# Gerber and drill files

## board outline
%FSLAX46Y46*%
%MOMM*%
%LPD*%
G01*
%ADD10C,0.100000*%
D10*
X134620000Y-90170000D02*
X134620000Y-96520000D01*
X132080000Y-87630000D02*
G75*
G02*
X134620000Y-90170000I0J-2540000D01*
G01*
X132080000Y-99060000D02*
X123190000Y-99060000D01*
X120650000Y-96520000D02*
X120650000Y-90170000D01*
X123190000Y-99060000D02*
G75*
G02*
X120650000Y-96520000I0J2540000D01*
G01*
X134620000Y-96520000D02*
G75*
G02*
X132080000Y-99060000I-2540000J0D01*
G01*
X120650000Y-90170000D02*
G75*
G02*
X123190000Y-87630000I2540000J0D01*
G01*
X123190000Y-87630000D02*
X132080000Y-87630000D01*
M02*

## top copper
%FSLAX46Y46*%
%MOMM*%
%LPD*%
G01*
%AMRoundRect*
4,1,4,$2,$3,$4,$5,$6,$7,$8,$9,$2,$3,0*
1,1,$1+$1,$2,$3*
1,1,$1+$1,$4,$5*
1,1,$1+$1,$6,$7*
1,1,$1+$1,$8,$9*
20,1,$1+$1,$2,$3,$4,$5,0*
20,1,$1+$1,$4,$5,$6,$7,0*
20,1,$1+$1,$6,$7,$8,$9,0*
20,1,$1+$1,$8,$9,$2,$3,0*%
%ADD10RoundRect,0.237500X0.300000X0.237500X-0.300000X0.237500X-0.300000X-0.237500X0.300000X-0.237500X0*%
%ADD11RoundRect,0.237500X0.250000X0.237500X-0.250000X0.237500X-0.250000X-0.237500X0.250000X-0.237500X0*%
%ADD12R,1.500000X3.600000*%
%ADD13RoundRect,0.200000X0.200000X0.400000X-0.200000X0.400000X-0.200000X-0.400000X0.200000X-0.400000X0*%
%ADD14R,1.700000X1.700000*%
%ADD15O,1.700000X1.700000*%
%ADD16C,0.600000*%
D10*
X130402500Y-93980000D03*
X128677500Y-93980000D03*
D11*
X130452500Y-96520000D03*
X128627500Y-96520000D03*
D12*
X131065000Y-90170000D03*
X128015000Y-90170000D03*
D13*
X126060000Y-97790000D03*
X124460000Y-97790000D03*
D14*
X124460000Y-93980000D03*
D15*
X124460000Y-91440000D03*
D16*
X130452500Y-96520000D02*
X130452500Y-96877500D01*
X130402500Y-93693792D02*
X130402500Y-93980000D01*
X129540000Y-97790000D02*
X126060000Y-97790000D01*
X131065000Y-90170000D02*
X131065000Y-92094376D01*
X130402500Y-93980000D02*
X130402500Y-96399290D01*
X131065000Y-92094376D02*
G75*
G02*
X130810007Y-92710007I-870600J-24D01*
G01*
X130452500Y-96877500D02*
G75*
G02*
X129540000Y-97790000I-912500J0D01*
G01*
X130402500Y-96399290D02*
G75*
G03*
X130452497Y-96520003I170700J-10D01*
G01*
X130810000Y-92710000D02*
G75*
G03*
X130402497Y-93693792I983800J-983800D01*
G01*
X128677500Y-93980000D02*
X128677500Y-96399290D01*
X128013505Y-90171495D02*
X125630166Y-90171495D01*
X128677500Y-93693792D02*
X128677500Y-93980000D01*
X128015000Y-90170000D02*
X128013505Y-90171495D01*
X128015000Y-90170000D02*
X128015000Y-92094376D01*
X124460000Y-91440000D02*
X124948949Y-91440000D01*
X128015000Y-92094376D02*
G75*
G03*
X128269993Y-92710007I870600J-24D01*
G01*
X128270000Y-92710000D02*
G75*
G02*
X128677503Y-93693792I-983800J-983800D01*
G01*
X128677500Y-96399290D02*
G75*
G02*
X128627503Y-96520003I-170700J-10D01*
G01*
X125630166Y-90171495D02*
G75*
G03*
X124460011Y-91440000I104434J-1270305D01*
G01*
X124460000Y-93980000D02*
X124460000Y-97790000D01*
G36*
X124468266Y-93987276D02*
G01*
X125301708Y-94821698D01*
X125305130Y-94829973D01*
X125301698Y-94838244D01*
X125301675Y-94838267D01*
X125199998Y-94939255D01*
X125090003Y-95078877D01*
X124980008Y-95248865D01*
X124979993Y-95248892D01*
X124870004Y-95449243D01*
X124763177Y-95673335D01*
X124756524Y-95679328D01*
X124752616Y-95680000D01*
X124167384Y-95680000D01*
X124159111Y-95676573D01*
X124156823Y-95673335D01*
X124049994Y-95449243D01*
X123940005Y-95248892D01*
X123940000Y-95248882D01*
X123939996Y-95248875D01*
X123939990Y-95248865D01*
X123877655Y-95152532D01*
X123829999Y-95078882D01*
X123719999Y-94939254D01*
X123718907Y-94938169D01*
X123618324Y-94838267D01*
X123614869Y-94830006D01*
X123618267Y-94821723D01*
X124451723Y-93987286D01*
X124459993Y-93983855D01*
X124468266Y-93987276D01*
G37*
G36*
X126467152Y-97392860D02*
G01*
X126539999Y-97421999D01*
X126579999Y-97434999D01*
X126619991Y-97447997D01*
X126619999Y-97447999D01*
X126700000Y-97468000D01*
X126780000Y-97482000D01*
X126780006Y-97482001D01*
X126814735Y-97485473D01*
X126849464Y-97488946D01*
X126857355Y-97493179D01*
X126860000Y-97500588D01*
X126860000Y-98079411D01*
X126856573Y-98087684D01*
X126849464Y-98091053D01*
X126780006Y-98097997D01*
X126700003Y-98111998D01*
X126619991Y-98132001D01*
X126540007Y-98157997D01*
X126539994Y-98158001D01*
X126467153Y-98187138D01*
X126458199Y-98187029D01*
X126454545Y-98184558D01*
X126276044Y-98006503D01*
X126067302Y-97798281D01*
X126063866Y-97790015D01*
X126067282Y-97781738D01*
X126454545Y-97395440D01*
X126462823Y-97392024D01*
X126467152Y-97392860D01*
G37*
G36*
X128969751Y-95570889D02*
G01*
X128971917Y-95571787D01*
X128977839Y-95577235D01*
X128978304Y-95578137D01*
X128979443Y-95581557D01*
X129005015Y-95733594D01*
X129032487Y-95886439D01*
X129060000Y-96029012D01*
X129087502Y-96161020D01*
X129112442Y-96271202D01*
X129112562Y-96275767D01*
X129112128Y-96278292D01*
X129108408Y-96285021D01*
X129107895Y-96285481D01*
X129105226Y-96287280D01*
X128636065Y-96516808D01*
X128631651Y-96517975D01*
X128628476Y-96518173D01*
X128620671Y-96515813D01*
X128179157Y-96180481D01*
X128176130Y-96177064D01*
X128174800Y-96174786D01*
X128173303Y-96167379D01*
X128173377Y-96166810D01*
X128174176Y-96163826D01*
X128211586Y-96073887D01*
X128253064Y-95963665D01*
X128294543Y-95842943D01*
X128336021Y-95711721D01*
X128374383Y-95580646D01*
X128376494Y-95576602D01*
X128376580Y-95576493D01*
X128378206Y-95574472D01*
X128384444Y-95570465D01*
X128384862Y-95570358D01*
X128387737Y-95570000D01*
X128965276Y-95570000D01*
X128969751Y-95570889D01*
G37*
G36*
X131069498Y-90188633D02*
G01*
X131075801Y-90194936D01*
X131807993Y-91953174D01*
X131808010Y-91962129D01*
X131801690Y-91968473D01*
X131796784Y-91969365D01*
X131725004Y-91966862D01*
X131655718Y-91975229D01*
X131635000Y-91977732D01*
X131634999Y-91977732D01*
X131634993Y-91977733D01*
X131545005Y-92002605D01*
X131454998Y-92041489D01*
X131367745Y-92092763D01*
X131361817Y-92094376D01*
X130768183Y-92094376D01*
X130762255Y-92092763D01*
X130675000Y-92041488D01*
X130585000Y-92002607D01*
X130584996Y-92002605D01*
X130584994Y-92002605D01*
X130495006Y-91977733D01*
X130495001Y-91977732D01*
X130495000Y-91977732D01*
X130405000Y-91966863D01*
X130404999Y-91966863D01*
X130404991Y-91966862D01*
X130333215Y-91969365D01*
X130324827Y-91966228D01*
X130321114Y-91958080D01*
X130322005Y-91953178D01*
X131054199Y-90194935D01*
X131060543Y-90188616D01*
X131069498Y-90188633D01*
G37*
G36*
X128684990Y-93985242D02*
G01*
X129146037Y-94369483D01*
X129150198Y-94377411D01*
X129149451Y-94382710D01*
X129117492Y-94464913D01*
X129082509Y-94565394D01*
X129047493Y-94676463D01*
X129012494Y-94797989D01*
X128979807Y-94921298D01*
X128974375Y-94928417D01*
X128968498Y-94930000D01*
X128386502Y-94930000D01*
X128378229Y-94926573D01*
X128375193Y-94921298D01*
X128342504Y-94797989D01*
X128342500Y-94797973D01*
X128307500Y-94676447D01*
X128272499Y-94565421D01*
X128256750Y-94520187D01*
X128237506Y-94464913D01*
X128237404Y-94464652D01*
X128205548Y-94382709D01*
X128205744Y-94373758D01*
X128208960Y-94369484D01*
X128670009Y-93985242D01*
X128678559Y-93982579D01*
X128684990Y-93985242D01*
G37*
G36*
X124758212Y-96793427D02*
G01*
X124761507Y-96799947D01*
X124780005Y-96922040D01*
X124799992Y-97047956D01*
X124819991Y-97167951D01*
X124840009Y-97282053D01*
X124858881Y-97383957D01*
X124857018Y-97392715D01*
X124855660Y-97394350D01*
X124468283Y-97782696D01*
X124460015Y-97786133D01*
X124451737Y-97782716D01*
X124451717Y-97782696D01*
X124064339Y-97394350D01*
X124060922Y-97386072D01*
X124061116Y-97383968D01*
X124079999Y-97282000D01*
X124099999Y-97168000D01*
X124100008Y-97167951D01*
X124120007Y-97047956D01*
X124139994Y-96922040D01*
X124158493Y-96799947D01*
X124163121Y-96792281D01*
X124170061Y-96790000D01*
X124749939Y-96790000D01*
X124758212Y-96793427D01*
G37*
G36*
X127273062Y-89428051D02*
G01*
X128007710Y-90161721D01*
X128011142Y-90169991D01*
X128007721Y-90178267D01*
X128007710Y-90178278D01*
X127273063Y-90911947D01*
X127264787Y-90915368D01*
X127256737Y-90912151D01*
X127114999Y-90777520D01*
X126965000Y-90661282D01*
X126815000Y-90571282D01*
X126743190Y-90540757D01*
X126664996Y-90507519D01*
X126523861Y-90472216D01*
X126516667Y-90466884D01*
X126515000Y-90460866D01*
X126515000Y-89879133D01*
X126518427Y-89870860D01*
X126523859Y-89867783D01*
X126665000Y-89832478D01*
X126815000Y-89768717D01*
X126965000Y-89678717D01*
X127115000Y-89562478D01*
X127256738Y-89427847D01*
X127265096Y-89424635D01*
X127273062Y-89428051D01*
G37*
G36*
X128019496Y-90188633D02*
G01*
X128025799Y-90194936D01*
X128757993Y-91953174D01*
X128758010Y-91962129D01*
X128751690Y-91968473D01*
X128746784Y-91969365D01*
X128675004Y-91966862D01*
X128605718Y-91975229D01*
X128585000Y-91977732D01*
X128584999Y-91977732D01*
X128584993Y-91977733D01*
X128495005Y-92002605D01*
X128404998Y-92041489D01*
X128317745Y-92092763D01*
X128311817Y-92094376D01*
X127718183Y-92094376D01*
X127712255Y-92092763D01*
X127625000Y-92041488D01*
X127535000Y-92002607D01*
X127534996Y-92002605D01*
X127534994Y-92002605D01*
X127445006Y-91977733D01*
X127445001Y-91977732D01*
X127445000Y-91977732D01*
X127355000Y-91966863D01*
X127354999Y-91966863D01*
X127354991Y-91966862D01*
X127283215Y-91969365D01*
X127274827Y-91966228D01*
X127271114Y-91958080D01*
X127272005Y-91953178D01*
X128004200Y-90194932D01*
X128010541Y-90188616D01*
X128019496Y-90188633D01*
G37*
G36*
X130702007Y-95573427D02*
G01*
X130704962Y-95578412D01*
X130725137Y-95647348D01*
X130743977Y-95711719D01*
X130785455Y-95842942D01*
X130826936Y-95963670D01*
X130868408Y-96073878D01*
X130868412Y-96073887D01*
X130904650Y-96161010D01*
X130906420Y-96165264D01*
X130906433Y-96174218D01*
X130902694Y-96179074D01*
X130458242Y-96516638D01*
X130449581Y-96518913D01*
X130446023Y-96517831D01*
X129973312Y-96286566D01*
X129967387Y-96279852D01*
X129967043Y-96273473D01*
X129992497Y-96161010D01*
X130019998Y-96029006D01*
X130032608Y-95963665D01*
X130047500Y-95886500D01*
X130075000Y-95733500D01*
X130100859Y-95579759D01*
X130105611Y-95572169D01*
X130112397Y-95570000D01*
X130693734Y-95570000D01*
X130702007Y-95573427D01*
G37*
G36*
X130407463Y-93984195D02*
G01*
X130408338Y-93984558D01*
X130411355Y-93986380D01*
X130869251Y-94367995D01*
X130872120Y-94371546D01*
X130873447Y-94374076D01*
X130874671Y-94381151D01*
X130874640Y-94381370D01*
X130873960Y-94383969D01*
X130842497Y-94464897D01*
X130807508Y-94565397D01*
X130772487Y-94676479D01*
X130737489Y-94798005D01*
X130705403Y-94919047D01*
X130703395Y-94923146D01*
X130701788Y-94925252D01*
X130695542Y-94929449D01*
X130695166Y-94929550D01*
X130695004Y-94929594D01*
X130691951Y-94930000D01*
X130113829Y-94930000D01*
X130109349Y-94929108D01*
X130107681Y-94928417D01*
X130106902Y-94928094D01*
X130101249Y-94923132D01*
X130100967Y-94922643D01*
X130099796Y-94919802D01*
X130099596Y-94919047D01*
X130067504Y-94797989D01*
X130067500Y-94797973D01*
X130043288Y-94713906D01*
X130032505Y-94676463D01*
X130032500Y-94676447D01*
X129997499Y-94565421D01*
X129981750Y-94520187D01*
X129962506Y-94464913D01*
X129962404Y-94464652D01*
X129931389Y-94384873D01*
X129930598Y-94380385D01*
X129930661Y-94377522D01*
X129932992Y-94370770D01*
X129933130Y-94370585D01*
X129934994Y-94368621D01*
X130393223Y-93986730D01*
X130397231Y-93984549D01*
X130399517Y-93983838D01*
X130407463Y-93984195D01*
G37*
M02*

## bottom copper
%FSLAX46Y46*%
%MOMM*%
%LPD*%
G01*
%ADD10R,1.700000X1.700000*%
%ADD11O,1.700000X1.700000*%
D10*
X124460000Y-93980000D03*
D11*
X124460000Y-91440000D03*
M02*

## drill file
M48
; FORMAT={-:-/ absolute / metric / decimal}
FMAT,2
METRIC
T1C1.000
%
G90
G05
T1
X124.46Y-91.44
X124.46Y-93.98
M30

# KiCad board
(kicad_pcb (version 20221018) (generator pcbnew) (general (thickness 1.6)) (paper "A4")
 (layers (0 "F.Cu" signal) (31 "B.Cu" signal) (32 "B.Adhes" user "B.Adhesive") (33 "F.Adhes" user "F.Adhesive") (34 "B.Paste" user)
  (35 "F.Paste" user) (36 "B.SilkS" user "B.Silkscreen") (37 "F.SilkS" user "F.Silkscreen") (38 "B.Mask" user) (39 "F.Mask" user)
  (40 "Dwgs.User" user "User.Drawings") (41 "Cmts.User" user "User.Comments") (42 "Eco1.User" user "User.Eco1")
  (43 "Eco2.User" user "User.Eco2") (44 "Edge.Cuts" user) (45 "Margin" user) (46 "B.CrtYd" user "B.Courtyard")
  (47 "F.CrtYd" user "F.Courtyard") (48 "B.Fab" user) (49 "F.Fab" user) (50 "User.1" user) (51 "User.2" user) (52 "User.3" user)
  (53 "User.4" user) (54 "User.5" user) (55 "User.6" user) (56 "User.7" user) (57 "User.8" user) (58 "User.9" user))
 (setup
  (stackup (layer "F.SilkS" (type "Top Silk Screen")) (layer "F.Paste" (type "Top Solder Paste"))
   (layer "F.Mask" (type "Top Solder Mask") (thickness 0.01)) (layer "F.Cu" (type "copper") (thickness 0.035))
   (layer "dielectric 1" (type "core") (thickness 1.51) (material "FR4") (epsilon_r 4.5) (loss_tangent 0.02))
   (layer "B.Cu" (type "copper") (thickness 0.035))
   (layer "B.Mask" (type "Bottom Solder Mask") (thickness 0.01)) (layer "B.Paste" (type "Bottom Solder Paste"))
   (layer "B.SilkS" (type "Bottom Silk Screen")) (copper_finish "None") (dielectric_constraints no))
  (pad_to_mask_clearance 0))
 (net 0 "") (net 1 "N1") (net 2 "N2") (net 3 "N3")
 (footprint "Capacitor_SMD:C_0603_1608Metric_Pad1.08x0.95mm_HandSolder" (layer "F.Cu") (at 129.54 93.98 180)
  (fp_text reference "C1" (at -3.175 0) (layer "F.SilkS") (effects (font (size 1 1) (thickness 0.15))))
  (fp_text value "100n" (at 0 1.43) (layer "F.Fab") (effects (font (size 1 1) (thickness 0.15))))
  (pad "1" smd roundrect (at -0.8625 0 180) (size 1.075 0.95) (layers "F.Cu" "F.Paste" "F.Mask") (roundrect_rratio 0.25) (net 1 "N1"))
  (pad "2" smd roundrect (at 0.8625 0 180) (size 1.075 0.95) (layers "F.Cu" "F.Paste" "F.Mask") (roundrect_rratio 0.25) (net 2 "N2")))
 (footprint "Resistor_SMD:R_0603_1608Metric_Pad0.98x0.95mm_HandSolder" (layer "F.Cu") (at 129.54 96.52 180)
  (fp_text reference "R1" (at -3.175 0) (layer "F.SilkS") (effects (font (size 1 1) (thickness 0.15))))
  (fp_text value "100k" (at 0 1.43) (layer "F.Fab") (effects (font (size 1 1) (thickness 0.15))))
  (pad "1" smd roundrect (at -0.9125 0 180) (size 0.975 0.95) (layers "F.Cu" "F.Paste" "F.Mask") (roundrect_rratio 0.25) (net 1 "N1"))
  (pad "2" smd roundrect (at 0.9125 0 180) (size 0.975 0.95) (layers "F.Cu" "F.Paste" "F.Mask") (roundrect_rratio 0.25) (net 2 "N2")))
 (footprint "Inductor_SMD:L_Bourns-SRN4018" (layer "F.Cu") (at 129.54 90.17 180)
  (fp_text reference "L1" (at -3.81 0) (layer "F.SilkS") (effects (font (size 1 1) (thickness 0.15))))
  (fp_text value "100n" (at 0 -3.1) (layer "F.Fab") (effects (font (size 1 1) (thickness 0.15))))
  (pad "1" smd rect (at -1.525 0 180) (size 1.5 3.6) (layers "F.Cu" "F.Paste" "F.Mask") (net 1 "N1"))
  (pad "2" smd rect (at 1.525 0 180) (size 1.5 3.6) (layers "F.Cu" "F.Paste" "F.Mask") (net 2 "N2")))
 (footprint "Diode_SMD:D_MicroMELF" (layer "F.Cu") (at 125.26 97.79 180)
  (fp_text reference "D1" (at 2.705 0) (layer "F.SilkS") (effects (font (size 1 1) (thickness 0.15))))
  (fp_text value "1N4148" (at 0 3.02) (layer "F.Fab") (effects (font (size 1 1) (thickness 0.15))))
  (pad "1" smd roundrect (at -0.8 0 180) (size 0.8 1.2) (layers "F.Cu" "F.Paste" "F.Mask") (roundrect_rratio 0.25) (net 1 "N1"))
  (pad "2" smd roundrect (at 0.8 0 180) (size 0.8 1.2) (layers "F.Cu" "F.Paste" "F.Mask") (roundrect_rratio 0.25) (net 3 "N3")))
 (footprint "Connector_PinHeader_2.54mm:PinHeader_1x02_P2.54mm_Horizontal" (layer "F.Cu") (at 124.46 93.98 180)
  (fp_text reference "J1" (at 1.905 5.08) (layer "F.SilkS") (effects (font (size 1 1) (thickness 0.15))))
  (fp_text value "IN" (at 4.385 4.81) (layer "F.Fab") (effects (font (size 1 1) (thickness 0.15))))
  (pad "1" thru_hole rect (at 0 0 180) (size 1.7 1.7) (drill 1) (layers "*.Cu" "*.Mask") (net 3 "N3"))
  (pad "2" thru_hole oval (at 0 2.54 180) (size 1.7 1.7) (drill 1) (layers "*.Cu" "*.Mask") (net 2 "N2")))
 (gr_line (start 134.62 90.17) (end 134.62 96.52) (stroke (width 0.1) (type default)) (layer "Edge.Cuts"))
 (gr_arc (start 132.08 87.63) (mid 133.876051 88.373949) (end 134.62 90.17) (stroke (width 0.1) (type default)) (layer "Edge.Cuts"))
 (gr_line (start 132.08 99.06) (end 123.19 99.06) (stroke (width 0.1) (type default)) (layer "Edge.Cuts"))
 (gr_line (start 120.65 96.52) (end 120.65 90.17) (stroke (width 0.1) (type default)) (layer "Edge.Cuts"))
 (gr_arc (start 123.19 99.06) (mid 121.393949 98.316051) (end 120.65 96.52) (stroke (width 0.1) (type default)) (layer "Edge.Cuts"))
 (gr_arc (start 134.62 96.52) (mid 133.876051 98.316051) (end 132.08 99.06) (stroke (width 0.1) (type default)) (layer "Edge.Cuts"))
 (gr_arc (start 120.65 90.17) (mid 121.393949 88.373949) (end 123.19 87.63) (stroke (width 0.1) (type default)) (layer "Edge.Cuts"))
 (gr_line (start 123.19 87.63) (end 132.08 87.63) (stroke (width 0.1) (type default)) (layer "Edge.Cuts"))
 (segment (start 130.4525 96.52) (end 130.4525 96.8775) (width 0.6) (layer "F.Cu") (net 1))
 (segment (start 130.4025 93.693792) (end 130.4025 93.98) (width 0.6) (layer "F.Cu") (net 1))
 (segment (start 129.54 97.79) (end 126.06 97.79) (width 0.6) (layer "F.Cu") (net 1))
 (segment (start 131.065 90.17) (end 131.065 92.094376) (width 0.6) (layer "F.Cu") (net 1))
 (segment (start 130.4025 93.98) (end 130.4025 96.39929) (width 0.6) (layer "F.Cu") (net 1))
 (arc (start 131.065 92.094376) (mid 130.998728 92.427549) (end 130.81 92.71) (width 0.6) (layer "F.Cu") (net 1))
 (arc (start 130.4525 96.8775) (mid 130.185235 97.522735) (end 129.54 97.79) (width 0.6) (layer "F.Cu") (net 1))
 (arc (start 130.4025 96.39929) (mid 130.415494 96.464618) (end 130.4525 96.52) (width 0.6) (layer "F.Cu") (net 1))
 (arc (start 130.81 92.71) (mid 130.508406 93.161367) (end 130.4025 93.693792) (width 0.6) (layer "F.Cu") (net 1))
 (segment (start 128.6775 93.98) (end 128.6775 96.39929) (width 0.6) (layer "F.Cu") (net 2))
 (segment (start 128.013505 90.171495) (end 125.630166 90.171495) (width 0.6) (layer "F.Cu") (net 2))
 (segment (start 128.6775 93.693792) (end 128.6775 93.98) (width 0.6) (layer "F.Cu") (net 2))
 (segment (start 128.015 90.17) (end 128.013505 90.171495) (width 0.6) (layer "F.Cu") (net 2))
 (segment (start 128.015 90.17) (end 128.015 92.094376) (width 0.6) (layer "F.Cu") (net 2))
 (segment (start 124.46 91.44) (end 124.948949 91.44) (width 0.6) (layer "F.Cu") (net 2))
 (arc (start 128.015 92.094376) (mid 128.081272 92.427549) (end 128.27 92.71) (width 0.6) (layer "F.Cu") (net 2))
 (arc (start 128.27 92.71) (mid 128.571594 93.161367) (end 128.6775 93.693792) (width 0.6) (layer "F.Cu") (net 2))
 (arc (start 128.6775 96.39929) (mid 128.664505 96.464617) (end 128.6275 96.52) (width 0.6) (layer "F.Cu") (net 2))
 (arc (start 125.630166 90.171495) (mid 124.79741 90.577923) (end 124.46 91.44) (width 0.6) (layer "F.Cu") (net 2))
 (segment (start 124.46 93.98) (end 124.46 97.79) (width 0.6) (layer "F.Cu") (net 3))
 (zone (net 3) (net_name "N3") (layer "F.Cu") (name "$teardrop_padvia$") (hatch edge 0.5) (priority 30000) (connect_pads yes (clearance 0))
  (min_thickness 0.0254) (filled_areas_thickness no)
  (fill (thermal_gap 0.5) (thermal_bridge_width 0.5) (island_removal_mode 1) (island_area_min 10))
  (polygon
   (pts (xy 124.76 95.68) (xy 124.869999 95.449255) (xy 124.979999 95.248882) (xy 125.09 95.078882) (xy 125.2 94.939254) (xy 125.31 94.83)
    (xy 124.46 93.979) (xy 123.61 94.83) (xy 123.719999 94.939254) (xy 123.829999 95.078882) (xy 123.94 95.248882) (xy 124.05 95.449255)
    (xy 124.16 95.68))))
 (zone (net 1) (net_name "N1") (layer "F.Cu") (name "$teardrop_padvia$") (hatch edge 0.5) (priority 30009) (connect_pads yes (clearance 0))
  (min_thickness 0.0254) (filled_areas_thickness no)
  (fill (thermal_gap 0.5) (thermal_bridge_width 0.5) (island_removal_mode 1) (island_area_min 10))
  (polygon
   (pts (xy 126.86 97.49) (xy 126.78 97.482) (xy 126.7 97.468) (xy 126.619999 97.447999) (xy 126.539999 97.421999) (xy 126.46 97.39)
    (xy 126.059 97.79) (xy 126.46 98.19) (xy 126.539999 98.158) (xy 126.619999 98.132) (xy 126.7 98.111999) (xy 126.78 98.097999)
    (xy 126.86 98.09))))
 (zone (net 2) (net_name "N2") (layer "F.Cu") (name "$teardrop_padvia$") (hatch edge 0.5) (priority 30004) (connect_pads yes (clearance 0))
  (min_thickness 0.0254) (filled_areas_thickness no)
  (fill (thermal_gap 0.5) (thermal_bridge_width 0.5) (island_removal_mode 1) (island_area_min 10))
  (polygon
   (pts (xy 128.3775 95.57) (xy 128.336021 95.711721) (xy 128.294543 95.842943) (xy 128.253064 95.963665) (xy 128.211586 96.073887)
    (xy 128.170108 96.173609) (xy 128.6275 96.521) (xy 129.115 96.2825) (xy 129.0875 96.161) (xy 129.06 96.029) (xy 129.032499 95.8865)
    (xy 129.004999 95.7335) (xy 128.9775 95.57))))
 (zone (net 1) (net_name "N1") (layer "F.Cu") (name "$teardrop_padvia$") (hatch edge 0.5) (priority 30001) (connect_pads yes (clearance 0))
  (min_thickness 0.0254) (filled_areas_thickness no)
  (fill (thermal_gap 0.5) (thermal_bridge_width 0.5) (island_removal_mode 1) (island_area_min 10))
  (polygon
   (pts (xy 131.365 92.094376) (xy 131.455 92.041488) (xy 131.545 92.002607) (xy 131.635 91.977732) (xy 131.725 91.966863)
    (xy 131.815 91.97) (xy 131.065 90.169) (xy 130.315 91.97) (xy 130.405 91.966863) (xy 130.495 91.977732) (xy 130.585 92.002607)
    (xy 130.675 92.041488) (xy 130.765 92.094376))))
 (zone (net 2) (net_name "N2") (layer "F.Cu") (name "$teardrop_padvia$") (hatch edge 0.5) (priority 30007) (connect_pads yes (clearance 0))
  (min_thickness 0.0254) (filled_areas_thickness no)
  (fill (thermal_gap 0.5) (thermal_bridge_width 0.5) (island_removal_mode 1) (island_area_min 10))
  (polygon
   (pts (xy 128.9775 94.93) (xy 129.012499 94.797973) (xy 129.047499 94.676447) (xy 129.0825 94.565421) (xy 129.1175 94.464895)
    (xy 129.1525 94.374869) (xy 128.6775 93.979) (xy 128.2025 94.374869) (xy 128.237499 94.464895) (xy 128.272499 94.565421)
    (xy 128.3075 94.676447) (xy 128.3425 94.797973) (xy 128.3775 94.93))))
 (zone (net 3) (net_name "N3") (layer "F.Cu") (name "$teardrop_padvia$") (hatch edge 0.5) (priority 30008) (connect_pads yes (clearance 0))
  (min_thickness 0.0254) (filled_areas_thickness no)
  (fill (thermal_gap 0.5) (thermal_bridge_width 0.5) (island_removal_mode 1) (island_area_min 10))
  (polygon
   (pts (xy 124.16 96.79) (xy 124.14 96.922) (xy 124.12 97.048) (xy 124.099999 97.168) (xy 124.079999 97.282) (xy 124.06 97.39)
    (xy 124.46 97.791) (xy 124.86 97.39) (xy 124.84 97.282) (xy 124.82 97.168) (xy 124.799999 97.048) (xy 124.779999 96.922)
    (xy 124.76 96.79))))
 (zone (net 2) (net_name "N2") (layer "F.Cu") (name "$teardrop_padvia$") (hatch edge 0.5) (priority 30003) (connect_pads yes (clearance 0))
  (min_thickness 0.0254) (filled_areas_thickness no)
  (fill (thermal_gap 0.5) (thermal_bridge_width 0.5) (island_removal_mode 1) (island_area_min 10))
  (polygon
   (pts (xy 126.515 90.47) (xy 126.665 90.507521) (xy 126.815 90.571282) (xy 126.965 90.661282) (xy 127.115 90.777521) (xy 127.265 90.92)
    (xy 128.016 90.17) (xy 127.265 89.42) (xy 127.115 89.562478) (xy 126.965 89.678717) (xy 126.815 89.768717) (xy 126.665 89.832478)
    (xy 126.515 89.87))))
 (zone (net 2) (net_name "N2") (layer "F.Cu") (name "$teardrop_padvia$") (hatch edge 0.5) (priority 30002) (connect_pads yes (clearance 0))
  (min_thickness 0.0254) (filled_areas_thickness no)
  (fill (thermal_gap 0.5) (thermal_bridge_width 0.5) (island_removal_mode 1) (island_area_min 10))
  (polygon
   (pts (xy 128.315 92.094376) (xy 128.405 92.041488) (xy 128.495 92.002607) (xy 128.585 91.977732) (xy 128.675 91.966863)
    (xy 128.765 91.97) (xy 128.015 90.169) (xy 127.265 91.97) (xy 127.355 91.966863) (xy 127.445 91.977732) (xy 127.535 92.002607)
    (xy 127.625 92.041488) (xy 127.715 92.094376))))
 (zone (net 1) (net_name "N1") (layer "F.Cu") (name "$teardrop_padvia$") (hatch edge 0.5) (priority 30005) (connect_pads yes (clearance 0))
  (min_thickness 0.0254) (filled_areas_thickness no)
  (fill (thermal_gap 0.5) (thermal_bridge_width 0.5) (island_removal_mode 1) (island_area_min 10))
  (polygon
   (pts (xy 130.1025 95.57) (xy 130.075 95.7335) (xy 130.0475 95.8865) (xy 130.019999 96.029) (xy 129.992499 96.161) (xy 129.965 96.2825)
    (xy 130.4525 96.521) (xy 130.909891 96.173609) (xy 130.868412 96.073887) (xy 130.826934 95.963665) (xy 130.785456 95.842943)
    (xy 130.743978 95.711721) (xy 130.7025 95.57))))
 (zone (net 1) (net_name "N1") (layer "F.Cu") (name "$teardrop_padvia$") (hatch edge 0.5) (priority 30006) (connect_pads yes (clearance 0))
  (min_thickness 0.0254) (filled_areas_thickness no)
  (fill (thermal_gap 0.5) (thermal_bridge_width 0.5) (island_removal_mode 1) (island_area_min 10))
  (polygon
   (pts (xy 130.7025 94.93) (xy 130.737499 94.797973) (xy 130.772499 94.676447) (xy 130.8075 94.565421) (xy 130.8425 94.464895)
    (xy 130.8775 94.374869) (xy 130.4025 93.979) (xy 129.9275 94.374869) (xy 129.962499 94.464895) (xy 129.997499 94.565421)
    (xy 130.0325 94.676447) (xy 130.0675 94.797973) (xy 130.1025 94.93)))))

